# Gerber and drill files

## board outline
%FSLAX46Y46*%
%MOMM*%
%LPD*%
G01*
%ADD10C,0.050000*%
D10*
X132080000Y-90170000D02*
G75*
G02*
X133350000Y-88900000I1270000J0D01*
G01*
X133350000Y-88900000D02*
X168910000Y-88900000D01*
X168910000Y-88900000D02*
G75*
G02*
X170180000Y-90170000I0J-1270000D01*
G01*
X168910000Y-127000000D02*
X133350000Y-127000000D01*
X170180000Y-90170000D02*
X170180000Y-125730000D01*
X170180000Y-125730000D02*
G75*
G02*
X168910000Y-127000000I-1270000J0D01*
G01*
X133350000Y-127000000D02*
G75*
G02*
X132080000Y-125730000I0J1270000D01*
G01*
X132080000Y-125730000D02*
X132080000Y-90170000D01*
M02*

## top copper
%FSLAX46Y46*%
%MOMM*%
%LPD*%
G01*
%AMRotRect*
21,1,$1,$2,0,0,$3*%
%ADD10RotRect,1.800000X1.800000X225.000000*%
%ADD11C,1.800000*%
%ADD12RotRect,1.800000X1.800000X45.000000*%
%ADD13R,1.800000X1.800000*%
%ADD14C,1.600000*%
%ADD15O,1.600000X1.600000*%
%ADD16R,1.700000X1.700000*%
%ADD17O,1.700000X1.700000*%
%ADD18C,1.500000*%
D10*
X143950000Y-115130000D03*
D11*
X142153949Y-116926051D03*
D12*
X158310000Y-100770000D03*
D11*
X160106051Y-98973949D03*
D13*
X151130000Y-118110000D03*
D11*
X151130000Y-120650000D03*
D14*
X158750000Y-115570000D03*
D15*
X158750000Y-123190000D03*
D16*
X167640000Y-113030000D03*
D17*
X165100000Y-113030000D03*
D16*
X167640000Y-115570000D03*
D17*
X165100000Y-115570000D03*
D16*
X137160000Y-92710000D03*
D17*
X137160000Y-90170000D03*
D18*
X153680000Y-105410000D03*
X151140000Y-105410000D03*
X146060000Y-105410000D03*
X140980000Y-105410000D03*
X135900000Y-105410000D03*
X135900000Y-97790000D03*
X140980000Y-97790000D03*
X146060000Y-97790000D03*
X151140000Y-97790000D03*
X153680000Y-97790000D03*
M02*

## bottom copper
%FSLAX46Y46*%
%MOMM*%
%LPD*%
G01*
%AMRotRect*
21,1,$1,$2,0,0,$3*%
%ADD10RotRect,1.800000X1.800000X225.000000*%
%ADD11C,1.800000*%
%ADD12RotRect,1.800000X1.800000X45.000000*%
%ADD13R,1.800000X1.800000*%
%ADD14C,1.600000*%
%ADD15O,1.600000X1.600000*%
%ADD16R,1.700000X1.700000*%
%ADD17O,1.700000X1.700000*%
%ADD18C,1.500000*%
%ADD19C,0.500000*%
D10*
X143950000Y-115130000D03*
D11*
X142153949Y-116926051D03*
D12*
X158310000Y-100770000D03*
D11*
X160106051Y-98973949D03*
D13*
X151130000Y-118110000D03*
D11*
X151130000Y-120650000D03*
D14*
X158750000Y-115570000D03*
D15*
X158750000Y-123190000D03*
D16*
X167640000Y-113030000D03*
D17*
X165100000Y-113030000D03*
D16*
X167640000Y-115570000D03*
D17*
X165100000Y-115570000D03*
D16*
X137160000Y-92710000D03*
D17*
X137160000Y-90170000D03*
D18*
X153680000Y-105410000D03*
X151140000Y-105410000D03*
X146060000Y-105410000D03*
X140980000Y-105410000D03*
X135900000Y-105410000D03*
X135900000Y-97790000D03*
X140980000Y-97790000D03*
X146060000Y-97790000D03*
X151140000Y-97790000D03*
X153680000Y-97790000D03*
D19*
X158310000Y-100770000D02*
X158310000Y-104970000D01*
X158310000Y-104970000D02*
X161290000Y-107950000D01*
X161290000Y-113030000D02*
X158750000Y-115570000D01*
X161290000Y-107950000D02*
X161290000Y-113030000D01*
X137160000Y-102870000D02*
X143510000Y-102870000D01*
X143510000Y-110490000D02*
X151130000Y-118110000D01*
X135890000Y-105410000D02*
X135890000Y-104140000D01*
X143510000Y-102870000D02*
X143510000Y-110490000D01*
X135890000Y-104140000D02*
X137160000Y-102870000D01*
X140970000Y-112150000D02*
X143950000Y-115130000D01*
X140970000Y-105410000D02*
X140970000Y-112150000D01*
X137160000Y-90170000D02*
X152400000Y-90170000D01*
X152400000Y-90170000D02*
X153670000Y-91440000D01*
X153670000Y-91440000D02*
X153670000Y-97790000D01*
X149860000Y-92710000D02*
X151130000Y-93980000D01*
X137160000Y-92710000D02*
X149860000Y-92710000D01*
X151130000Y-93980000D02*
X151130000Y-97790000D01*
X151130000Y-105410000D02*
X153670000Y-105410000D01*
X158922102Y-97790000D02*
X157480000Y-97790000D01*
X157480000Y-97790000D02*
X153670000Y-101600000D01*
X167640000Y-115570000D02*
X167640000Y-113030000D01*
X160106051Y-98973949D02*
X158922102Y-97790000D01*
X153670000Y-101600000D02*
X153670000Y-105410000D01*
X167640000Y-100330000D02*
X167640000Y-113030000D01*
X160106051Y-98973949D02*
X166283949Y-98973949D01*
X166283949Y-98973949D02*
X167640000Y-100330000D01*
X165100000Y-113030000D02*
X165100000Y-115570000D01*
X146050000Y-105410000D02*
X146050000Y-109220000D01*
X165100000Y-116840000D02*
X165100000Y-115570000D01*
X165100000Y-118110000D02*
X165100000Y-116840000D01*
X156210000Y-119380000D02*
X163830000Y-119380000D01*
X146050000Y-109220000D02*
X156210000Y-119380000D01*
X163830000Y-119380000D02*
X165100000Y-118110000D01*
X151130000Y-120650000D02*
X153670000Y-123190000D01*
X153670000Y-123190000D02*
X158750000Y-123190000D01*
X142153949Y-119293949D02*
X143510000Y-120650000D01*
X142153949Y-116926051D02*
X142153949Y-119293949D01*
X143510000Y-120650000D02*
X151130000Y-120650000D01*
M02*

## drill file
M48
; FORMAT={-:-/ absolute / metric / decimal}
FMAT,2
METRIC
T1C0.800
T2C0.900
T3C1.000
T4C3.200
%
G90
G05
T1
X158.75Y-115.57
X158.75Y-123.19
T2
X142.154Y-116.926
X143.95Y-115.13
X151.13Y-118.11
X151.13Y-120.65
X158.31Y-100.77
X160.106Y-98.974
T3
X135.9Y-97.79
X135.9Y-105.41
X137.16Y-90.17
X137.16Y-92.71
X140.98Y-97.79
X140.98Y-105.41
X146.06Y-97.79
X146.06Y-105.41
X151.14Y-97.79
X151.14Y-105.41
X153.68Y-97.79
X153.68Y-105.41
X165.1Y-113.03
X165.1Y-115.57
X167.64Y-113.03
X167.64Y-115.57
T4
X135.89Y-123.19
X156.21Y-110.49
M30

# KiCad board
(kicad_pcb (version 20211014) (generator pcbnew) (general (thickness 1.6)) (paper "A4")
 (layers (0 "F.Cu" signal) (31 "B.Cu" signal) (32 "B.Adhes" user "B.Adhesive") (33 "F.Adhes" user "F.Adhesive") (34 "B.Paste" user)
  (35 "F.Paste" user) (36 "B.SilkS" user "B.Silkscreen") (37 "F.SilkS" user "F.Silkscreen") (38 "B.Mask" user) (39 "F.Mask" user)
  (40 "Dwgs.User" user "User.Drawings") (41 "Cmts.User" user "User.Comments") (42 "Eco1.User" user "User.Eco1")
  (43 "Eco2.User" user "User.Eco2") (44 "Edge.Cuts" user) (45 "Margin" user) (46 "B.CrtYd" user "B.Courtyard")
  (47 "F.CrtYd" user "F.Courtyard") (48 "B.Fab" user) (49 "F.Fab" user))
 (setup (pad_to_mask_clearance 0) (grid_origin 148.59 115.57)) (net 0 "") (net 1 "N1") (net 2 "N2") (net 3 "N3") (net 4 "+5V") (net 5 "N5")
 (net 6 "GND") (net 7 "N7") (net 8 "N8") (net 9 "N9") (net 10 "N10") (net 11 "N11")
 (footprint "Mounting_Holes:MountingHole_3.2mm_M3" (layer "F.Cu") (at 156.21 110.49 -90)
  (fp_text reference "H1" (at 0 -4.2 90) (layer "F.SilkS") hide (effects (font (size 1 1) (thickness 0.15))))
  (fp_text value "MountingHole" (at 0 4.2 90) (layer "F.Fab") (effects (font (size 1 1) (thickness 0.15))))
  (pad "" np_thru_hole circle locked (at 0 0 270) (size 3.2 3.2) (drill 3.2) (layers *.Cu *.Mask) (thermal_gap 2)))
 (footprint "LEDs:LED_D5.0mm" (layer "F.Cu") (at 143.95 115.13 -135)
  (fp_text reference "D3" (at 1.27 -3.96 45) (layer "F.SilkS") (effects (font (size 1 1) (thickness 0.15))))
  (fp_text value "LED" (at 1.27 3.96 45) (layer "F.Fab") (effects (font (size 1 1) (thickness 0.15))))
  (pad "1" thru_hole rect locked (at 0 0 225) (size 1.8 1.8) (drill 0.9) (layers *.Cu *.Mask) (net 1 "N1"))
  (pad "2" thru_hole circle locked (at 2.54 0 225) (size 1.8 1.8) (drill 0.9) (layers *.Cu *.Mask) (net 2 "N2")))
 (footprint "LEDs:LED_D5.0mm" (layer "F.Cu") (at 158.31 100.77 45)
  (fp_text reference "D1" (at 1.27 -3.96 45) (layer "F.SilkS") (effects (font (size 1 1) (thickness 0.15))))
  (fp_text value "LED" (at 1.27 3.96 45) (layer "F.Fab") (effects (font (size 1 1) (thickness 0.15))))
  (pad "1" thru_hole rect locked (at 0 0 45) (size 1.8 1.8) (drill 0.9) (layers *.Cu *.Mask) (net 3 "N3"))
  (pad "2" thru_hole circle locked (at 2.54 0 45) (size 1.8 1.8) (drill 0.9) (layers *.Cu *.Mask) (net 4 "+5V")))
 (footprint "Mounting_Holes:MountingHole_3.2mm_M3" (layer "F.Cu") (at 135.89 123.19 -90)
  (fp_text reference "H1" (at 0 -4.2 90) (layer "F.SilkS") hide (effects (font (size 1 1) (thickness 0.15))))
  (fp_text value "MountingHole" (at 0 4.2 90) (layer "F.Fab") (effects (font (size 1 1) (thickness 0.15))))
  (pad "" np_thru_hole circle locked (at 0 0 270) (size 3.2 3.2) (drill 3.2) (layers *.Cu *.Mask) (thermal_gap 2)))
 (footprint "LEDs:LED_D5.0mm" (layer "F.Cu") (at 151.13 118.11 -90)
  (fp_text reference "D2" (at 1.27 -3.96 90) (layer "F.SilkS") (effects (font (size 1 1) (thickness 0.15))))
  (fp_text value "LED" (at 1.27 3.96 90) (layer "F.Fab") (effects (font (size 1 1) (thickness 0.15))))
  (pad "1" thru_hole rect locked (at 0 0 270) (size 1.8 1.8) (drill 0.9) (layers *.Cu *.Mask) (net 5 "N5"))
  (pad "2" thru_hole circle locked (at 2.54 0 270) (size 1.8 1.8) (drill 0.9) (layers *.Cu *.Mask) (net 2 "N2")))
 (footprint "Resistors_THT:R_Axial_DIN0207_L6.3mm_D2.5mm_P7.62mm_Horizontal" (layer "F.Cu") (at 158.75 115.57 -90)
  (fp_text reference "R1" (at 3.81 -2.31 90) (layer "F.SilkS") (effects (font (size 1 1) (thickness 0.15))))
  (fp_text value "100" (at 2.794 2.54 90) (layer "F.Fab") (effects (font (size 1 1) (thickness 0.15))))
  (pad "1" thru_hole circle locked (at 0 0 270) (size 1.6 1.6) (drill 0.8) (layers *.Cu *.Mask) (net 3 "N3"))
  (pad "2" thru_hole oval locked (at 7.62 0 270) (size 1.6 1.6) (drill 0.8) (layers *.Cu *.Mask) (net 2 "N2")))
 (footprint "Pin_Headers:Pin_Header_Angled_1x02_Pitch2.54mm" (layer "B.Cu") (at 167.64 113.03 90)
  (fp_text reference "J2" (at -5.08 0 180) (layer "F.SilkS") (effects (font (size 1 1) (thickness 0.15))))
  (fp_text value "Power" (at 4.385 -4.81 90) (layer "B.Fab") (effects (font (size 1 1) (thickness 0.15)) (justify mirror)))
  (pad "1" thru_hole rect locked (at 0 0 90) (size 1.7 1.7) (drill 1) (layers *.Cu *.Mask) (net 4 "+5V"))
  (pad "2" thru_hole oval locked (at 0 -2.54 90) (size 1.7 1.7) (drill 1) (layers *.Cu *.Mask) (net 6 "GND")))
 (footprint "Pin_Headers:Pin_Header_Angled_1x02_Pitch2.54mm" (layer "B.Cu") (at 167.64 115.57 90)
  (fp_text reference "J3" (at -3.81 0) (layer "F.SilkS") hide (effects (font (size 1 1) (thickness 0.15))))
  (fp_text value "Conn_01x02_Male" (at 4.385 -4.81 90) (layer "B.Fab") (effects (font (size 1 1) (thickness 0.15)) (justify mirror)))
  (pad "1" thru_hole rect locked (at 0 0 90) (size 1.7 1.7) (drill 1) (layers *.Cu *.Mask) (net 4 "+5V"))
  (pad "2" thru_hole oval locked (at 0 -2.54 90) (size 1.7 1.7) (drill 1) (layers *.Cu *.Mask) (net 6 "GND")))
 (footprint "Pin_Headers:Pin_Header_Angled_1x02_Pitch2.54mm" (layer "B.Cu") (at 137.16 92.71)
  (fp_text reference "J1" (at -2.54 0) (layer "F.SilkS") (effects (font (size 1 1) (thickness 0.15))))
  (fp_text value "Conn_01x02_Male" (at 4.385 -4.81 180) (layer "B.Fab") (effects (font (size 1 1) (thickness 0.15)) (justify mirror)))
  (pad "1" thru_hole rect locked (at 0 0) (size 1.7 1.7) (drill 1) (layers *.Cu *.Mask) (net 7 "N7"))
  (pad "2" thru_hole oval locked (at 0 -2.54) (size 1.7 1.7) (drill 1) (layers *.Cu *.Mask) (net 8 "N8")))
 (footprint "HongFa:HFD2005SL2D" (layer "B.Cu") (at 153.68 105.41 180)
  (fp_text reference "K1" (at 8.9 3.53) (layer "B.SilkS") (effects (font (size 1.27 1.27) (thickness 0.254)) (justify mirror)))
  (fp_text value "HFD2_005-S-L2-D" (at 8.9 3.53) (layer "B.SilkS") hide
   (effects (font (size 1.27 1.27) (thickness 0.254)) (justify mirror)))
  (pad "1" thru_hole circle locked (at 0 0 180) (size 1.5 1.5) (drill 1) (layers *.Cu *.Mask) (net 4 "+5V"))
  (pad "2" thru_hole circle locked (at 2.54 0 180) (size 1.5 1.5) (drill 1) (layers *.Cu *.Mask) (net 4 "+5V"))
  (pad "4" thru_hole circle locked (at 7.62 0 180) (size 1.5 1.5) (drill 1) (layers *.Cu *.Mask) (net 6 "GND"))
  (pad "6" thru_hole circle locked (at 12.7 0 180) (size 1.5 1.5) (drill 1) (layers *.Cu *.Mask) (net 1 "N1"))
  (pad "8" thru_hole circle locked (at 17.78 0 180) (size 1.5 1.5) (drill 1) (layers *.Cu *.Mask) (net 5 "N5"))
  (pad "9" thru_hole circle locked (at 17.78 7.62 180) (size 1.5 1.5) (drill 1) (layers *.Cu *.Mask) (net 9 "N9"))
  (pad "11" thru_hole circle locked (at 12.7 7.62 180) (size 1.5 1.5) (drill 1) (layers *.Cu *.Mask) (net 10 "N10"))
  (pad "13" thru_hole circle locked (at 7.62 7.62 180) (size 1.5 1.5) (drill 1) (layers *.Cu *.Mask) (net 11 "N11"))
  (pad "15" thru_hole circle locked (at 2.54 7.62 180) (size 1.5 1.5) (drill 1) (layers *.Cu *.Mask) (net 7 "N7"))
  (pad "16" thru_hole circle locked (at 0 7.62 180) (size 1.5 1.5) (drill 1) (layers *.Cu *.Mask) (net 8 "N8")))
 (gr_arc (start 132.08 90.17) (mid 132.451974 89.271974) (end 133.35 88.9) (layer "Edge.Cuts") (width 0.05))
 (gr_line (start 133.35 88.9) (end 168.91 88.9) (layer "Edge.Cuts") (width 0.05))
 (gr_arc (start 168.91 88.9) (mid 169.808026 89.271974) (end 170.18 90.17) (layer "Edge.Cuts") (width 0.05))
 (gr_line (start 168.91 127) (end 133.35 127) (layer "Edge.Cuts") (width 0.05))
 (gr_line (start 170.18 90.17) (end 170.18 125.73) (layer "Edge.Cuts") (width 0.05))
 (gr_arc (start 170.18 125.73) (mid 169.808026 126.628026) (end 168.91 127) (layer "Edge.Cuts") (width 0.05))
 (gr_arc (start 133.35 127) (mid 132.451974 126.628026) (end 132.08 125.73) (layer "Edge.Cuts") (width 0.05))
 (gr_line (start 132.08 125.73) (end 132.08 90.17) (layer "Edge.Cuts") (width 0.05))
 (segment (start 158.31 100.77) (end 158.31 104.97) (width 0.5) (layer "B.Cu") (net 3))
 (segment (start 158.31 104.97) (end 161.29 107.95) (width 0.5) (layer "B.Cu") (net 3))
 (segment (start 161.29 113.03) (end 158.75 115.57) (width 0.5) (layer "B.Cu") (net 3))
 (segment (start 161.29 107.95) (end 161.29 113.03) (width 0.5) (layer "B.Cu") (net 3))
 (segment (start 137.16 102.87) (end 143.51 102.87) (width 0.5) (layer "B.Cu") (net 5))
 (segment (start 143.51 110.49) (end 151.13 118.11) (width 0.5) (layer "B.Cu") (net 5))
 (segment (start 135.89 105.41) (end 135.89 104.14) (width 0.5) (layer "B.Cu") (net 5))
 (segment (start 143.51 102.87) (end 143.51 110.49) (width 0.5) (layer "B.Cu") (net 5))
 (segment (start 135.89 104.14) (end 137.16 102.87) (width 0.5) (layer "B.Cu") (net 5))
 (segment (start 140.97 112.15) (end 143.95 115.13) (width 0.5) (layer "B.Cu") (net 1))
 (segment (start 140.97 105.41) (end 140.97 112.15) (width 0.5) (layer "B.Cu") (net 1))
 (segment (start 137.16 90.17) (end 152.4 90.17) (width 0.5) (layer "B.Cu") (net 8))
 (segment (start 152.4 90.17) (end 153.67 91.44) (width 0.5) (layer "B.Cu") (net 8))
 (segment (start 153.67 91.44) (end 153.67 97.79) (width 0.5) (layer "B.Cu") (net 8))
 (segment (start 149.86 92.71) (end 151.13 93.98) (width 0.5) (layer "B.Cu") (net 7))
 (segment (start 137.16 92.71) (end 149.86 92.71) (width 0.5) (layer "B.Cu") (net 7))
 (segment (start 151.13 93.98) (end 151.13 97.79) (width 0.5) (layer "B.Cu") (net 7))
 (segment (start 151.13 105.41) (end 153.67 105.41) (width 0.5) (layer "B.Cu") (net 4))
 (segment (start 158.922102 97.79) (end 157.48 97.79) (width 0.5) (layer "B.Cu") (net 4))
 (segment (start 157.48 97.79) (end 153.67 101.6) (width 0.5) (layer "B.Cu") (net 4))
 (segment (start 167.64 115.57) (end 167.64 113.03) (width 0.5) (layer "B.Cu") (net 4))
 (segment (start 160.106051 98.973949) (end 158.922102 97.79) (width 0.5) (layer "B.Cu") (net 4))
 (segment (start 153.67 101.6) (end 153.67 105.41) (width 0.5) (layer "B.Cu") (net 4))
 (segment (start 167.64 100.33) (end 167.64 113.03) (width 0.5) (layer "B.Cu") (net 4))
 (segment (start 160.106051 98.973949) (end 166.283949 98.973949) (width 0.5) (layer "B.Cu") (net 4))
 (segment (start 166.283949 98.973949) (end 167.64 100.33) (width 0.5) (layer "B.Cu") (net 4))
 (segment (start 165.1 113.03) (end 165.1 115.57) (width 0.5) (layer "B.Cu") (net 6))
 (segment (start 146.05 105.41) (end 146.05 109.22) (width 0.5) (layer "B.Cu") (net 6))
 (segment (start 165.1 116.84) (end 165.1 115.57) (width 0.5) (layer "B.Cu") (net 6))
 (segment (start 165.1 118.11) (end 165.1 116.84) (width 0.5) (layer "B.Cu") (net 6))
 (segment (start 156.21 119.38) (end 163.83 119.38) (width 0.5) (layer "B.Cu") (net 6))
 (segment (start 146.05 109.22) (end 156.21 119.38) (width 0.5) (layer "B.Cu") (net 6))
 (segment (start 163.83 119.38) (end 165.1 118.11) (width 0.5) (layer "B.Cu") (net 6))
 (segment (start 151.13 120.65) (end 153.67 123.19) (width 0.5) (layer "B.Cu") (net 2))
 (segment (start 153.67 123.19) (end 158.75 123.19) (width 0.5) (layer "B.Cu") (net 2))
 (segment (start 142.153949 119.293949) (end 143.51 120.65) (width 0.5) (layer "B.Cu") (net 2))
 (segment (start 142.153949 116.926051) (end 142.153949 119.293949) (width 0.5) (layer "B.Cu") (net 2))
 (segment (start 143.51 120.65) (end 151.13 120.65) (width 0.5) (layer "B.Cu") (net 2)))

